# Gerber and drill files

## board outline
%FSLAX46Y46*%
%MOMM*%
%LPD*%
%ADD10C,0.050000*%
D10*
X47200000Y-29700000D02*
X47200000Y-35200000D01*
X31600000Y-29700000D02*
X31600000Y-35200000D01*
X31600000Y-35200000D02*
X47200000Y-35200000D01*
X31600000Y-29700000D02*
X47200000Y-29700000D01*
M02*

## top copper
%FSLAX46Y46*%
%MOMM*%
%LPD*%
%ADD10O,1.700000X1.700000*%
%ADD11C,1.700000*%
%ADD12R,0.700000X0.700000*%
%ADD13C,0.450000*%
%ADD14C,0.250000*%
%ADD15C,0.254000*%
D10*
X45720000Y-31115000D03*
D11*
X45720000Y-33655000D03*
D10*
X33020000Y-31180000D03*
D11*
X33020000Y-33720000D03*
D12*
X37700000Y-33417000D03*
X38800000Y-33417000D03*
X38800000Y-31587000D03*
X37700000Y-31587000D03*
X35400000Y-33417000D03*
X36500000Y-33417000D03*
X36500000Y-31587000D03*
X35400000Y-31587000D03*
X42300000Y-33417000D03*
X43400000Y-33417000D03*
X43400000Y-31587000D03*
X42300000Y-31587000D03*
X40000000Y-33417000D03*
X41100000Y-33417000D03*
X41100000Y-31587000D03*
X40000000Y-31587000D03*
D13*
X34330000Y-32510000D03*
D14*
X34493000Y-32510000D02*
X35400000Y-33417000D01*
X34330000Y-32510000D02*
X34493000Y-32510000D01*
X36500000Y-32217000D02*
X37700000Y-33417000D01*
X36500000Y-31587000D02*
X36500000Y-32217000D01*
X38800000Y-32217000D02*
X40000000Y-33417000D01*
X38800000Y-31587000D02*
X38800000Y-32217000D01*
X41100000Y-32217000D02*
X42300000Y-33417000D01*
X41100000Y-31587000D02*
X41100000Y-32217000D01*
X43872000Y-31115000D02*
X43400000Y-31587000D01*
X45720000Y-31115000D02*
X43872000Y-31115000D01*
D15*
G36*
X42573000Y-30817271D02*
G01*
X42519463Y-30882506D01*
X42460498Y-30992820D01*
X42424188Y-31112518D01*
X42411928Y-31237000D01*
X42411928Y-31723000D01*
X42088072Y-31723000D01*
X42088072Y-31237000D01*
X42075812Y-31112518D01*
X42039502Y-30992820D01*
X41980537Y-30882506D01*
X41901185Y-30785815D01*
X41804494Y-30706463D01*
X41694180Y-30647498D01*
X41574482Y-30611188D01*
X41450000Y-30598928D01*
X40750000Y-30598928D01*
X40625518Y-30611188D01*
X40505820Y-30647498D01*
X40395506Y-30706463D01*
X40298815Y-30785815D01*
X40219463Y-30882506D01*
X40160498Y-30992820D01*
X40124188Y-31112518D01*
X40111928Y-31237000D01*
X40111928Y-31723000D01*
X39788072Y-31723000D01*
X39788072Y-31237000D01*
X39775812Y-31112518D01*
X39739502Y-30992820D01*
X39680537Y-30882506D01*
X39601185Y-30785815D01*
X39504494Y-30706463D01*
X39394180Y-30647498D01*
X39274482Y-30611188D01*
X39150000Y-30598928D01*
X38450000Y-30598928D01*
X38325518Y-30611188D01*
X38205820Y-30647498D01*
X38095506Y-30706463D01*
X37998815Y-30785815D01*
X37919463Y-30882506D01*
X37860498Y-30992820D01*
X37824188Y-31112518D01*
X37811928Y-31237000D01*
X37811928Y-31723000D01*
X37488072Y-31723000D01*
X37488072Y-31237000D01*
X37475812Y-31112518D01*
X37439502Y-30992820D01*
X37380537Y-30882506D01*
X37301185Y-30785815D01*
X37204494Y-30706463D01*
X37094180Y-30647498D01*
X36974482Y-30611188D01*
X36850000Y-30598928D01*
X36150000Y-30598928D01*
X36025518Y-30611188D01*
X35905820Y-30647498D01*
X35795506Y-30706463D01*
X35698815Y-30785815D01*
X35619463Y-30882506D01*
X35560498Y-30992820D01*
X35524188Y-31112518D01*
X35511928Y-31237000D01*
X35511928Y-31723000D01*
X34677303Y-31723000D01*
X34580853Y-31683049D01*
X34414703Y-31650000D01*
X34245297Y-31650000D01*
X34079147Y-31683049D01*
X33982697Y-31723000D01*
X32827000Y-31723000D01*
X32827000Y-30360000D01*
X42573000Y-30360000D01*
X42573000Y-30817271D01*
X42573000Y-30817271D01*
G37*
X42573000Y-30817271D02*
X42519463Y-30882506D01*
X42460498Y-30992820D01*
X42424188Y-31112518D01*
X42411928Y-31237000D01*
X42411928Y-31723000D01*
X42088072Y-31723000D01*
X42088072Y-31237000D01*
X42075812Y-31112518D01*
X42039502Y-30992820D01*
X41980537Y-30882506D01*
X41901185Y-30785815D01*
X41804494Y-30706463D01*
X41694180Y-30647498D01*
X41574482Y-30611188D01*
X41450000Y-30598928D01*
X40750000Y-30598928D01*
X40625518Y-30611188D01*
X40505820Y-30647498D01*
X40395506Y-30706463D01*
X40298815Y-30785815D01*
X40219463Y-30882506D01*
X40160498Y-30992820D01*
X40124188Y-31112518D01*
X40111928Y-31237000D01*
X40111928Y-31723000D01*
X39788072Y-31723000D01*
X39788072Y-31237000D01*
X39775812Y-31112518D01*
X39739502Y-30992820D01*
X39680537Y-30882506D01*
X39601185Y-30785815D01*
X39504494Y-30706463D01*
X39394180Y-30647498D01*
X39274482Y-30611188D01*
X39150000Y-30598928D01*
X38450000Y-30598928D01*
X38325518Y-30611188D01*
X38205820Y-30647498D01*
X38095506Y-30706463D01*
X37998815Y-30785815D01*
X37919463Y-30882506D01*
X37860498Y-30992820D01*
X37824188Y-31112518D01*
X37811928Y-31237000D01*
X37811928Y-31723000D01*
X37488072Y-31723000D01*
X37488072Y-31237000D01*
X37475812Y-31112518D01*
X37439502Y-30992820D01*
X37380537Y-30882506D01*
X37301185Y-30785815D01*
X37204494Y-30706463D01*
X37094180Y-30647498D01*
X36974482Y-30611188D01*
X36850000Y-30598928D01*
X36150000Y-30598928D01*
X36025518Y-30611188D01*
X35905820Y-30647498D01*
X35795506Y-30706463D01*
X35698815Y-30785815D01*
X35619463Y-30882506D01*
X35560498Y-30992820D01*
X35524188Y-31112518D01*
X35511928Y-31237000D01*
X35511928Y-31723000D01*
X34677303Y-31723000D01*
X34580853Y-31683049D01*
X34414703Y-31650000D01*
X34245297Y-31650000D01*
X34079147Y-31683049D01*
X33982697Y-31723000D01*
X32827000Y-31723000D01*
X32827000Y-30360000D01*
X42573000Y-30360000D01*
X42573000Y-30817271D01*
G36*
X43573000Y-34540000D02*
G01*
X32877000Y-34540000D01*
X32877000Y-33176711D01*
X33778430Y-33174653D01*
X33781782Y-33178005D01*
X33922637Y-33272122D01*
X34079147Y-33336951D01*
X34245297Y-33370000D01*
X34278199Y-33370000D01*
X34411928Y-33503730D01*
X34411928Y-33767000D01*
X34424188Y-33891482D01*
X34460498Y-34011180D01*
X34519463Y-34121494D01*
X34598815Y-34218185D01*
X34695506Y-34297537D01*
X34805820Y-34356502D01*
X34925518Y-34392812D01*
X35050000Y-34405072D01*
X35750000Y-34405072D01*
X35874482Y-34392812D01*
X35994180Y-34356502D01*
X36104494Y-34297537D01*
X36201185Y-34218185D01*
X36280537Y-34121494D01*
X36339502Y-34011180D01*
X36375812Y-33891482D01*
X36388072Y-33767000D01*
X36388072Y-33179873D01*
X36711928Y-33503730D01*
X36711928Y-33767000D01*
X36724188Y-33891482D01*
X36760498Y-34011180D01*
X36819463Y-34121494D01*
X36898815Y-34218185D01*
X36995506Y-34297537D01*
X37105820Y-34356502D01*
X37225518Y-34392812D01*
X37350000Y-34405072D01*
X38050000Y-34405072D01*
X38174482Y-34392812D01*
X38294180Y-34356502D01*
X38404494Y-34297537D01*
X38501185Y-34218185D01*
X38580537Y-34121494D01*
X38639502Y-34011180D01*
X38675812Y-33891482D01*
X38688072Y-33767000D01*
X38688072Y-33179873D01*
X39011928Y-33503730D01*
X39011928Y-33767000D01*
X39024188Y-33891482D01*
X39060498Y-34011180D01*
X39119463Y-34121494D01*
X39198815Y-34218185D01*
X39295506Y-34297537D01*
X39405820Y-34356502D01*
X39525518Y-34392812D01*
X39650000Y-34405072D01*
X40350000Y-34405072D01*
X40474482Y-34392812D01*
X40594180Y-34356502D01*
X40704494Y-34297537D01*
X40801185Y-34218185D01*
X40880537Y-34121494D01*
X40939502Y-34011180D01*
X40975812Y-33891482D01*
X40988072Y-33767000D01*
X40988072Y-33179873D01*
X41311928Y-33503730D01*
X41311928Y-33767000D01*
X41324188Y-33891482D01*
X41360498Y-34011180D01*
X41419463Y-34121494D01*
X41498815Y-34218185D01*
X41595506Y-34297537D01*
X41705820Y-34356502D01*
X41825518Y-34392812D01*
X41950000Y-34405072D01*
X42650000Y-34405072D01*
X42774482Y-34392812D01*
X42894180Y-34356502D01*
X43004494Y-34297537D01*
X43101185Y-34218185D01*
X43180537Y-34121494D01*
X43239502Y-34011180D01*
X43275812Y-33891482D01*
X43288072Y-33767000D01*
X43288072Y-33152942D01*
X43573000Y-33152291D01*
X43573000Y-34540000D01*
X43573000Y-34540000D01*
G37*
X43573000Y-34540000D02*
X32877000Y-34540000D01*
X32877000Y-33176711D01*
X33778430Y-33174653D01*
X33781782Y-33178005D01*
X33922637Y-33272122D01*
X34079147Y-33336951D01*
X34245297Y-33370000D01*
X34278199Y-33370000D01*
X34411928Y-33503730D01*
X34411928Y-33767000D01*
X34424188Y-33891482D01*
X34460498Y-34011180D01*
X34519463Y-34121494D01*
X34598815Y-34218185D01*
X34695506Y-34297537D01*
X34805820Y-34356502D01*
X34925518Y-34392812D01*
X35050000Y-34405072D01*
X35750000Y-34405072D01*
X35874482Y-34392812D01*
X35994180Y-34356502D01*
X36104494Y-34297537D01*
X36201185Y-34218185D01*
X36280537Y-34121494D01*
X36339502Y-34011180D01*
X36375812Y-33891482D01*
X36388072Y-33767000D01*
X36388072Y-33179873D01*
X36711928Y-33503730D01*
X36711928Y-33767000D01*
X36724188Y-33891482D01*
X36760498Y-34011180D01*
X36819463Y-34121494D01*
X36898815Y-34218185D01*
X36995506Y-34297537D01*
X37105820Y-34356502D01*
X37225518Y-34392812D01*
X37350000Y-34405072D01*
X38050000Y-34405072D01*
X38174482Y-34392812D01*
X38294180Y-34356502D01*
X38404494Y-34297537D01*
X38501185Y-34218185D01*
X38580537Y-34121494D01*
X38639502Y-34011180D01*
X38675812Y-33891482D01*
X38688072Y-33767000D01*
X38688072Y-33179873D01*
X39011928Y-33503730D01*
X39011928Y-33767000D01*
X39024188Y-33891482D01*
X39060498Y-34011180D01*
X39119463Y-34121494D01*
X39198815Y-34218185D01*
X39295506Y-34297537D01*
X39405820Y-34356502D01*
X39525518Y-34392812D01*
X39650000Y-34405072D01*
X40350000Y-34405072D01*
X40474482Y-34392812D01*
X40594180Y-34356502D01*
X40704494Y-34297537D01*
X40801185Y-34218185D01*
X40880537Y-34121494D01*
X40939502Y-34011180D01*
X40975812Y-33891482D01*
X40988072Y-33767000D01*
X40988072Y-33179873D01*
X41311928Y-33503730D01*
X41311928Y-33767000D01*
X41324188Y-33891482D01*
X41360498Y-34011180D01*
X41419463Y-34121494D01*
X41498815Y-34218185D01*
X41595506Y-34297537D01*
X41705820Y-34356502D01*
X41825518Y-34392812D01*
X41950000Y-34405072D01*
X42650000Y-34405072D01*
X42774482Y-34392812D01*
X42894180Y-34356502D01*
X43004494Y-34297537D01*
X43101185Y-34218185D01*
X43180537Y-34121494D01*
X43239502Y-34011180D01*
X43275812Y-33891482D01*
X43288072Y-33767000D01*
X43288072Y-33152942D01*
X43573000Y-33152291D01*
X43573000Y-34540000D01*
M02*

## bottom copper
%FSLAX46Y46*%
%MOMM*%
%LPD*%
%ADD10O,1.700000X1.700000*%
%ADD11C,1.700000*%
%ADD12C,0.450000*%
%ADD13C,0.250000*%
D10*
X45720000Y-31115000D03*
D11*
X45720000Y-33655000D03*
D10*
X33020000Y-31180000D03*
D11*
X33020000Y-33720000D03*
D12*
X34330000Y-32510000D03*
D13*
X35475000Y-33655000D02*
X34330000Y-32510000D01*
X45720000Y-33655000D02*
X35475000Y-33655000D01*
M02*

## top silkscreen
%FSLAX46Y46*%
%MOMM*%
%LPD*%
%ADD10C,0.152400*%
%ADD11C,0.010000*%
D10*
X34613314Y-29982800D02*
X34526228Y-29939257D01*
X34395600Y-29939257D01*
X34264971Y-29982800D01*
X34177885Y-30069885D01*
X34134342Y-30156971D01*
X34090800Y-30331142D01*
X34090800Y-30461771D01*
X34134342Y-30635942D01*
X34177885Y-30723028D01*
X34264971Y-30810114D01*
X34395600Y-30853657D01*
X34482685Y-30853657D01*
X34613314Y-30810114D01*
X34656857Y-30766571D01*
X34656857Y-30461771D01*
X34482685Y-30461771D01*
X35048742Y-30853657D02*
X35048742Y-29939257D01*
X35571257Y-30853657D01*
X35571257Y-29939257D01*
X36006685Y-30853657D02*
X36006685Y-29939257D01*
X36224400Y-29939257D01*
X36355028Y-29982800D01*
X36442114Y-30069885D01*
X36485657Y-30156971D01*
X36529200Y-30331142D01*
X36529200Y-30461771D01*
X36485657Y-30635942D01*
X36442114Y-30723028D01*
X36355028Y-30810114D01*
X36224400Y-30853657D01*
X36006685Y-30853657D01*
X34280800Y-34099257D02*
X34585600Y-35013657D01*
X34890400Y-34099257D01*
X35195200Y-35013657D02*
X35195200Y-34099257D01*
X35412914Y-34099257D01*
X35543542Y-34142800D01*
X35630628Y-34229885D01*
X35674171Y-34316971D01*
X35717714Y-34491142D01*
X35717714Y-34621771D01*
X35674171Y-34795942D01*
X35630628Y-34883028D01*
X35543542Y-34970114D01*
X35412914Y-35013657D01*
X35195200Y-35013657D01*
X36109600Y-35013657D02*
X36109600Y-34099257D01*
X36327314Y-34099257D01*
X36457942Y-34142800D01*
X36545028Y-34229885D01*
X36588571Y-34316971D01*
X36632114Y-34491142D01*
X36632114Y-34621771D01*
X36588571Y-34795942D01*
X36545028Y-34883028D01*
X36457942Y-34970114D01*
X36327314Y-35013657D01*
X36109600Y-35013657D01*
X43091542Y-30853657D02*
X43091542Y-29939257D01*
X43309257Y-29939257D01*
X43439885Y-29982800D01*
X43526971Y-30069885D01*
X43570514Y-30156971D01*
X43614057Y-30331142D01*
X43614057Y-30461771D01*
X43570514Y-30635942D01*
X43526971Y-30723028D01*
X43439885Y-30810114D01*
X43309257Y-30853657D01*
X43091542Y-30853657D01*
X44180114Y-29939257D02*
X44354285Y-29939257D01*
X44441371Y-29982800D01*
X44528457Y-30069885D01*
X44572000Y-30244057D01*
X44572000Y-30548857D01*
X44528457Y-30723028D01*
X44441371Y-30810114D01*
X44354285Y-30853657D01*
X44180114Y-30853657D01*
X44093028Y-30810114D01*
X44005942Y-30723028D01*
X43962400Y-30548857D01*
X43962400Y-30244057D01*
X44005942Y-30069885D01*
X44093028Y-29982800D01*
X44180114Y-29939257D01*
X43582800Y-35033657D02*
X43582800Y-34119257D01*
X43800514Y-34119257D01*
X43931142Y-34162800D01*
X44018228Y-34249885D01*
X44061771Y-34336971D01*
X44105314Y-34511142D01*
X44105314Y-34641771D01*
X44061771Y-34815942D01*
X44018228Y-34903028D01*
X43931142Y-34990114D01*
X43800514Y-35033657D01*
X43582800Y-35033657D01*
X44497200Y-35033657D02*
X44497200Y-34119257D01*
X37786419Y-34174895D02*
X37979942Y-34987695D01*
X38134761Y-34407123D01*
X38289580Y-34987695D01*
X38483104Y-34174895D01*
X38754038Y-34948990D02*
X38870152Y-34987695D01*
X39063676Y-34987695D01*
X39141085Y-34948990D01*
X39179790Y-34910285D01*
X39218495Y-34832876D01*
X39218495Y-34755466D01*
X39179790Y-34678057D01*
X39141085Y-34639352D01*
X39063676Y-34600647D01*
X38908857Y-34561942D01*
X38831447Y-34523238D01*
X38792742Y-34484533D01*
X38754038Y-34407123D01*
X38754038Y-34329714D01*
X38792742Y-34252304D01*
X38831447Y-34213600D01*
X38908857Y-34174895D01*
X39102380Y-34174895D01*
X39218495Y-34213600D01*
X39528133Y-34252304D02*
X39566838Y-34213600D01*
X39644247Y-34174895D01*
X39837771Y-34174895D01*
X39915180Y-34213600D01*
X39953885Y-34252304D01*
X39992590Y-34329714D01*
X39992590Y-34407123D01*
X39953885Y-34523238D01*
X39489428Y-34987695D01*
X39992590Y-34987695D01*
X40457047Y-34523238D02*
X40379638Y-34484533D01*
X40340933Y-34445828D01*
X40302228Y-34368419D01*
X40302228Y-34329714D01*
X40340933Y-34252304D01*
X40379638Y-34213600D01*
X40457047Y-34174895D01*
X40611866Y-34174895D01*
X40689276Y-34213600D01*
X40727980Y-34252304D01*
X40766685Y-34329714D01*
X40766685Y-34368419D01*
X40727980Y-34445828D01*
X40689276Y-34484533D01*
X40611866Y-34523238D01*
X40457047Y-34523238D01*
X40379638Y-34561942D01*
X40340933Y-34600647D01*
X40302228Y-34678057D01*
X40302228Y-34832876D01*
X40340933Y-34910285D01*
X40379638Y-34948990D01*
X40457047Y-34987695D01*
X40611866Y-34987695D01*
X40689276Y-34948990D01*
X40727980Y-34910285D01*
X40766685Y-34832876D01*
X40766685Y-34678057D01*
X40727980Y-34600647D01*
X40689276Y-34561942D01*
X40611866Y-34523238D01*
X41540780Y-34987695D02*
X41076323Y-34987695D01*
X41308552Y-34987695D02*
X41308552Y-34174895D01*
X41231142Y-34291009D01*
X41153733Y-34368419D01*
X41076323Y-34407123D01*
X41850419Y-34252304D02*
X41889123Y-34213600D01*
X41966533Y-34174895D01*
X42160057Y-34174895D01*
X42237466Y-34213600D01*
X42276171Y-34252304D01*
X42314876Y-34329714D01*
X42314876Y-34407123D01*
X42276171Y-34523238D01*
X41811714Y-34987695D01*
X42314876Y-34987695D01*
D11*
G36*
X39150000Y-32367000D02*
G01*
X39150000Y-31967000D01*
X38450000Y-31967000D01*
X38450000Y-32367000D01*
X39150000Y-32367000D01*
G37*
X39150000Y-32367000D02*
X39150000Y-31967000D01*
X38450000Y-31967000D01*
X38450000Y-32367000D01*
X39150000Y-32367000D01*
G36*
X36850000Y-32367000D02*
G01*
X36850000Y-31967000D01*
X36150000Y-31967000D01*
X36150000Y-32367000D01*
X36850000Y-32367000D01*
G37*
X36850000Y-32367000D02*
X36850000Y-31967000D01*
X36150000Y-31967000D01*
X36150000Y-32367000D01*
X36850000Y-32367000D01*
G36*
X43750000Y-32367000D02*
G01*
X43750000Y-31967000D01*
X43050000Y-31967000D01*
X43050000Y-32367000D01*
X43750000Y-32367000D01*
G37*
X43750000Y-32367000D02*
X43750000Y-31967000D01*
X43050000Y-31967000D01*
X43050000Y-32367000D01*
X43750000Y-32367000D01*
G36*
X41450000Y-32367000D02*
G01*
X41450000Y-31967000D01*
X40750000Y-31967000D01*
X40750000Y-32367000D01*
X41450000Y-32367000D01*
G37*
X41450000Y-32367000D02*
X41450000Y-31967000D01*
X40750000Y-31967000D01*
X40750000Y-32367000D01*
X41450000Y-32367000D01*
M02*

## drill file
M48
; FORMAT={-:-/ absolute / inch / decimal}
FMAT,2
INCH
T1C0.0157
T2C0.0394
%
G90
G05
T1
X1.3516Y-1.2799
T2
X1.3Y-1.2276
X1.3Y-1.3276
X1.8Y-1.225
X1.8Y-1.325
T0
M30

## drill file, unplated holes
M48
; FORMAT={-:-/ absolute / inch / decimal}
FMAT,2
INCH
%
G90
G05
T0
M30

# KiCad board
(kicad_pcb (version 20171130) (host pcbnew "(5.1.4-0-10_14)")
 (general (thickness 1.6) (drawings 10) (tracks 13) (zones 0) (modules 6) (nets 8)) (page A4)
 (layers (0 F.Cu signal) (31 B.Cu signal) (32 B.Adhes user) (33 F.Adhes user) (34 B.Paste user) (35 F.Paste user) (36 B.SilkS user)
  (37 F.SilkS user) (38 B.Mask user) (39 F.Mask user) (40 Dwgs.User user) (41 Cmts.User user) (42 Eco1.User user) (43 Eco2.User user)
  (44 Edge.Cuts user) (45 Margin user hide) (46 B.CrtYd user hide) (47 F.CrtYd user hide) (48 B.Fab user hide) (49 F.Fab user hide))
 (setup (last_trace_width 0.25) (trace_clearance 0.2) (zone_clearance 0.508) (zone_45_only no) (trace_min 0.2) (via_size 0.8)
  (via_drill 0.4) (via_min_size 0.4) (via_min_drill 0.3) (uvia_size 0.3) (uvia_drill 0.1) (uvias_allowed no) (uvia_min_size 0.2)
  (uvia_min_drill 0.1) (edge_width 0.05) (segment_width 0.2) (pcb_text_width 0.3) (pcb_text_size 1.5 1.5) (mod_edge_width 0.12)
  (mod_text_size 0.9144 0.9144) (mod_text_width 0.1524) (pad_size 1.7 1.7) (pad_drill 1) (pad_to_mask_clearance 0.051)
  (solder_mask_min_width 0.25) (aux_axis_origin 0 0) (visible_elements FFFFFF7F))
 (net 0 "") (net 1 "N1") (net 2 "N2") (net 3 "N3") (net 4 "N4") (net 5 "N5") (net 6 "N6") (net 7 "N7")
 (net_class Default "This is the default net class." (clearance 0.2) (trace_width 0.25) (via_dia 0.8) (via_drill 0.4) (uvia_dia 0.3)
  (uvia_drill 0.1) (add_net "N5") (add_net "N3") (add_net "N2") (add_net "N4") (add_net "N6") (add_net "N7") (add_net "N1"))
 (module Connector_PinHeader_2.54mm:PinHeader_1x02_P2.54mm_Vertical (layer B.Cu) (at 45.72 33.655)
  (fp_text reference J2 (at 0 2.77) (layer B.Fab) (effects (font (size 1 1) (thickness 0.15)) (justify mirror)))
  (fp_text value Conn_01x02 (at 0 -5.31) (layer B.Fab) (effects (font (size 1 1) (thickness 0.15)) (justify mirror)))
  (pad 2 thru_hole oval (at 0 -2.54) (size 1.7 1.7) (drill 1) (layers *.Cu *.Mask) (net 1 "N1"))
  (pad 1 thru_hole circle (at 0 0) (size 1.7 1.7) (drill 1) (layers *.Cu *.Mask) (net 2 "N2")))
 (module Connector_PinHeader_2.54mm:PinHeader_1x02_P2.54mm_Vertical (layer B.Cu) (at 33.02 33.72)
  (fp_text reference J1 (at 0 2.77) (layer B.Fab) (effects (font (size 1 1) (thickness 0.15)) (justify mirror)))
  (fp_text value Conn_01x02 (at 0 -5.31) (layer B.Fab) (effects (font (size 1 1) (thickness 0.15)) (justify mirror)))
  (pad 2 thru_hole oval (at 0 -2.54) (size 1.7 1.7) (drill 1) (layers *.Cu *.Mask) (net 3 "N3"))
  (pad 1 thru_hole circle (at 0 0) (size 1.7 1.7) (drill 1) (layers *.Cu *.Mask) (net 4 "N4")))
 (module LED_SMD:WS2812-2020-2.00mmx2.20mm (layer F.Cu) (at 37.25 33.767 90)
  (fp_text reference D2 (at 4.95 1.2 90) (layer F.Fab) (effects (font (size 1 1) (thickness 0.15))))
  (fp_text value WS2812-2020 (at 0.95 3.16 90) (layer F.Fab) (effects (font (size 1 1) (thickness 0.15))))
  (fp_poly (pts (xy 1.4 1.9) (xy 1.8 1.9) (xy 1.8 1.2) (xy 1.4 1.2)) (layer F.SilkS) (width 0.01))
  (pad 3 smd rect (at 0.35 0.45 90) (size 0.7 0.7) (layers F.Cu F.Paste F.Mask) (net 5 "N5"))
  (pad 4 smd rect (at 0.35 1.55 90) (size 0.7 0.7) (layers F.Cu F.Paste F.Mask) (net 4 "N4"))
  (pad 1 smd rect (at 2.18 1.55 90) (size 0.7 0.7) (layers F.Cu F.Paste F.Mask) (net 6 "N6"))
  (pad 2 smd rect (at 2.18 0.45 90) (size 0.7 0.7) (layers F.Cu F.Paste F.Mask) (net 3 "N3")))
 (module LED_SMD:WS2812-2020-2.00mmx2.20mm (layer F.Cu) (at 34.95 33.767 90)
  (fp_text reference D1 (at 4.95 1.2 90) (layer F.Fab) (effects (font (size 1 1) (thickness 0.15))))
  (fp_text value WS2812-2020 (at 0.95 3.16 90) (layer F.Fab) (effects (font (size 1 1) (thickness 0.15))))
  (fp_poly (pts (xy 1.4 1.9) (xy 1.8 1.9) (xy 1.8 1.2) (xy 1.4 1.2)) (layer F.SilkS) (width 0.01))
  (pad 3 smd rect (at 0.35 0.45 90) (size 0.7 0.7) (layers F.Cu F.Paste F.Mask) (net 2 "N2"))
  (pad 4 smd rect (at 0.35 1.55 90) (size 0.7 0.7) (layers F.Cu F.Paste F.Mask) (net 4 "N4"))
  (pad 1 smd rect (at 2.18 1.55 90) (size 0.7 0.7) (layers F.Cu F.Paste F.Mask) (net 5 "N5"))
  (pad 2 smd rect (at 2.18 0.45 90) (size 0.7 0.7) (layers F.Cu F.Paste F.Mask) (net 3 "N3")))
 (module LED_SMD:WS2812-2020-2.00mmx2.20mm (layer F.Cu) (at 41.85 33.767 90)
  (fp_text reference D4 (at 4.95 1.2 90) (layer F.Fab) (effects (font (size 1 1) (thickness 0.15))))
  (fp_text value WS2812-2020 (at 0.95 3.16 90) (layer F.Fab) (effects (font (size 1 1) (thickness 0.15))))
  (fp_poly (pts (xy 1.4 1.9) (xy 1.8 1.9) (xy 1.8 1.2) (xy 1.4 1.2)) (layer F.SilkS) (width 0.01))
  (pad 3 smd rect (at 0.35 0.45 90) (size 0.7 0.7) (layers F.Cu F.Paste F.Mask) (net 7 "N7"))
  (pad 4 smd rect (at 0.35 1.55 90) (size 0.7 0.7) (layers F.Cu F.Paste F.Mask) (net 4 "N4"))
  (pad 1 smd rect (at 2.18 1.55 90) (size 0.7 0.7) (layers F.Cu F.Paste F.Mask) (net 1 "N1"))
  (pad 2 smd rect (at 2.18 0.45 90) (size 0.7 0.7) (layers F.Cu F.Paste F.Mask) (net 3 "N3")))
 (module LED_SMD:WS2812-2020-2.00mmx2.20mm (layer F.Cu) (at 39.55 33.767 90)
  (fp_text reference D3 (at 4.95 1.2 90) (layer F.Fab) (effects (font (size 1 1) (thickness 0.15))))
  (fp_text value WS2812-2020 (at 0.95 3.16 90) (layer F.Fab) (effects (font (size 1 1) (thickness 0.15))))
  (fp_poly (pts (xy 1.4 1.9) (xy 1.8 1.9) (xy 1.8 1.2) (xy 1.4 1.2)) (layer F.SilkS) (width 0.01))
  (pad 3 smd rect (at 0.35 0.45 90) (size 0.7 0.7) (layers F.Cu F.Paste F.Mask) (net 6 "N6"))
  (pad 4 smd rect (at 0.35 1.55 90) (size 0.7 0.7) (layers F.Cu F.Paste F.Mask) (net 4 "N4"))
  (pad 1 smd rect (at 2.18 1.55 90) (size 0.7 0.7) (layers F.Cu F.Paste F.Mask) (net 7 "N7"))
  (pad 2 smd rect (at 2.18 0.45 90) (size 0.7 0.7) (layers F.Cu F.Paste F.Mask) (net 3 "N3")))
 (gr_line (start 47.2 29.7) (end 47.2 35.2) (layer Edge.Cuts) (width 0.05))
 (gr_line (start 31.6 29.7) (end 31.6 35.2) (layer Edge.Cuts) (width 0.05))
 (gr_line (start 31.6 35.2) (end 47.2 35.2) (layer Edge.Cuts) (width 0.05))
 (gr_line (start 31.6 29.7) (end 47.2 29.7) (layer Edge.Cuts) (width 0.05))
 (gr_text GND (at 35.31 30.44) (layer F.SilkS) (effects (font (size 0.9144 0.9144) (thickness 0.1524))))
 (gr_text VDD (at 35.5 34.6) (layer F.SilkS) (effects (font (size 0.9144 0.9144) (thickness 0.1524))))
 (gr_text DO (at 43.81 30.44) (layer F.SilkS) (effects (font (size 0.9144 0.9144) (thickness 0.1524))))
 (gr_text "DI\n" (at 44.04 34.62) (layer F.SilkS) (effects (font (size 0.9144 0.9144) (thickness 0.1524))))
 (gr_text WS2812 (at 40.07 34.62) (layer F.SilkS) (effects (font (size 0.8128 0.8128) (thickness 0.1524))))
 (via blind (at 34.33 32.51) (size 0.45) (drill 0.4) (layers F.Cu B.Cu) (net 2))
 (segment (start 34.493 32.51) (end 35.4 33.417) (width 0.25) (layer F.Cu) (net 2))
 (segment (start 34.33 32.51) (end 34.493 32.51) (width 0.25) (layer F.Cu) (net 2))
 (segment (start 35.475 33.655) (end 34.33 32.51) (width 0.25) (layer B.Cu) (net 2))
 (segment (start 45.72 33.655) (end 35.475 33.655) (width 0.25) (layer B.Cu) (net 2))
 (segment (start 36.5 32.217) (end 37.7 33.417) (width 0.25) (layer F.Cu) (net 5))
 (segment (start 36.5 31.587) (end 36.5 32.217) (width 0.25) (layer F.Cu) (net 5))
 (segment (start 38.8 32.217) (end 40 33.417) (width 0.25) (layer F.Cu) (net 6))
 (segment (start 38.8 31.587) (end 38.8 32.217) (width 0.25) (layer F.Cu) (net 6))
 (segment (start 41.1 32.217) (end 42.3 33.417) (width 0.25) (layer F.Cu) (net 7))
 (segment (start 41.1 31.587) (end 41.1 32.217) (width 0.25) (layer F.Cu) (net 7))
 (segment (start 43.872 31.115) (end 43.4 31.587) (width 0.25) (layer F.Cu) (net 1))
 (segment (start 45.72 31.115) (end 43.872 31.115) (width 0.25) (layer F.Cu) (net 1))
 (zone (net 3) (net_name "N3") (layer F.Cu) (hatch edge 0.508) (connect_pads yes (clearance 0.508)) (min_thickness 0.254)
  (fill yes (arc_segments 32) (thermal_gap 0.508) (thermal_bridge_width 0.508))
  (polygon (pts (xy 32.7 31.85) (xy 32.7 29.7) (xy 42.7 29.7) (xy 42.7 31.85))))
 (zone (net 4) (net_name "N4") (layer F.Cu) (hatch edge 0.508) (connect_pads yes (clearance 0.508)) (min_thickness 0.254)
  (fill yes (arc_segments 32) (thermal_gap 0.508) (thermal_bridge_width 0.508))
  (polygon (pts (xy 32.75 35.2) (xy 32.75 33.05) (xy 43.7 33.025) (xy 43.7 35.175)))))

